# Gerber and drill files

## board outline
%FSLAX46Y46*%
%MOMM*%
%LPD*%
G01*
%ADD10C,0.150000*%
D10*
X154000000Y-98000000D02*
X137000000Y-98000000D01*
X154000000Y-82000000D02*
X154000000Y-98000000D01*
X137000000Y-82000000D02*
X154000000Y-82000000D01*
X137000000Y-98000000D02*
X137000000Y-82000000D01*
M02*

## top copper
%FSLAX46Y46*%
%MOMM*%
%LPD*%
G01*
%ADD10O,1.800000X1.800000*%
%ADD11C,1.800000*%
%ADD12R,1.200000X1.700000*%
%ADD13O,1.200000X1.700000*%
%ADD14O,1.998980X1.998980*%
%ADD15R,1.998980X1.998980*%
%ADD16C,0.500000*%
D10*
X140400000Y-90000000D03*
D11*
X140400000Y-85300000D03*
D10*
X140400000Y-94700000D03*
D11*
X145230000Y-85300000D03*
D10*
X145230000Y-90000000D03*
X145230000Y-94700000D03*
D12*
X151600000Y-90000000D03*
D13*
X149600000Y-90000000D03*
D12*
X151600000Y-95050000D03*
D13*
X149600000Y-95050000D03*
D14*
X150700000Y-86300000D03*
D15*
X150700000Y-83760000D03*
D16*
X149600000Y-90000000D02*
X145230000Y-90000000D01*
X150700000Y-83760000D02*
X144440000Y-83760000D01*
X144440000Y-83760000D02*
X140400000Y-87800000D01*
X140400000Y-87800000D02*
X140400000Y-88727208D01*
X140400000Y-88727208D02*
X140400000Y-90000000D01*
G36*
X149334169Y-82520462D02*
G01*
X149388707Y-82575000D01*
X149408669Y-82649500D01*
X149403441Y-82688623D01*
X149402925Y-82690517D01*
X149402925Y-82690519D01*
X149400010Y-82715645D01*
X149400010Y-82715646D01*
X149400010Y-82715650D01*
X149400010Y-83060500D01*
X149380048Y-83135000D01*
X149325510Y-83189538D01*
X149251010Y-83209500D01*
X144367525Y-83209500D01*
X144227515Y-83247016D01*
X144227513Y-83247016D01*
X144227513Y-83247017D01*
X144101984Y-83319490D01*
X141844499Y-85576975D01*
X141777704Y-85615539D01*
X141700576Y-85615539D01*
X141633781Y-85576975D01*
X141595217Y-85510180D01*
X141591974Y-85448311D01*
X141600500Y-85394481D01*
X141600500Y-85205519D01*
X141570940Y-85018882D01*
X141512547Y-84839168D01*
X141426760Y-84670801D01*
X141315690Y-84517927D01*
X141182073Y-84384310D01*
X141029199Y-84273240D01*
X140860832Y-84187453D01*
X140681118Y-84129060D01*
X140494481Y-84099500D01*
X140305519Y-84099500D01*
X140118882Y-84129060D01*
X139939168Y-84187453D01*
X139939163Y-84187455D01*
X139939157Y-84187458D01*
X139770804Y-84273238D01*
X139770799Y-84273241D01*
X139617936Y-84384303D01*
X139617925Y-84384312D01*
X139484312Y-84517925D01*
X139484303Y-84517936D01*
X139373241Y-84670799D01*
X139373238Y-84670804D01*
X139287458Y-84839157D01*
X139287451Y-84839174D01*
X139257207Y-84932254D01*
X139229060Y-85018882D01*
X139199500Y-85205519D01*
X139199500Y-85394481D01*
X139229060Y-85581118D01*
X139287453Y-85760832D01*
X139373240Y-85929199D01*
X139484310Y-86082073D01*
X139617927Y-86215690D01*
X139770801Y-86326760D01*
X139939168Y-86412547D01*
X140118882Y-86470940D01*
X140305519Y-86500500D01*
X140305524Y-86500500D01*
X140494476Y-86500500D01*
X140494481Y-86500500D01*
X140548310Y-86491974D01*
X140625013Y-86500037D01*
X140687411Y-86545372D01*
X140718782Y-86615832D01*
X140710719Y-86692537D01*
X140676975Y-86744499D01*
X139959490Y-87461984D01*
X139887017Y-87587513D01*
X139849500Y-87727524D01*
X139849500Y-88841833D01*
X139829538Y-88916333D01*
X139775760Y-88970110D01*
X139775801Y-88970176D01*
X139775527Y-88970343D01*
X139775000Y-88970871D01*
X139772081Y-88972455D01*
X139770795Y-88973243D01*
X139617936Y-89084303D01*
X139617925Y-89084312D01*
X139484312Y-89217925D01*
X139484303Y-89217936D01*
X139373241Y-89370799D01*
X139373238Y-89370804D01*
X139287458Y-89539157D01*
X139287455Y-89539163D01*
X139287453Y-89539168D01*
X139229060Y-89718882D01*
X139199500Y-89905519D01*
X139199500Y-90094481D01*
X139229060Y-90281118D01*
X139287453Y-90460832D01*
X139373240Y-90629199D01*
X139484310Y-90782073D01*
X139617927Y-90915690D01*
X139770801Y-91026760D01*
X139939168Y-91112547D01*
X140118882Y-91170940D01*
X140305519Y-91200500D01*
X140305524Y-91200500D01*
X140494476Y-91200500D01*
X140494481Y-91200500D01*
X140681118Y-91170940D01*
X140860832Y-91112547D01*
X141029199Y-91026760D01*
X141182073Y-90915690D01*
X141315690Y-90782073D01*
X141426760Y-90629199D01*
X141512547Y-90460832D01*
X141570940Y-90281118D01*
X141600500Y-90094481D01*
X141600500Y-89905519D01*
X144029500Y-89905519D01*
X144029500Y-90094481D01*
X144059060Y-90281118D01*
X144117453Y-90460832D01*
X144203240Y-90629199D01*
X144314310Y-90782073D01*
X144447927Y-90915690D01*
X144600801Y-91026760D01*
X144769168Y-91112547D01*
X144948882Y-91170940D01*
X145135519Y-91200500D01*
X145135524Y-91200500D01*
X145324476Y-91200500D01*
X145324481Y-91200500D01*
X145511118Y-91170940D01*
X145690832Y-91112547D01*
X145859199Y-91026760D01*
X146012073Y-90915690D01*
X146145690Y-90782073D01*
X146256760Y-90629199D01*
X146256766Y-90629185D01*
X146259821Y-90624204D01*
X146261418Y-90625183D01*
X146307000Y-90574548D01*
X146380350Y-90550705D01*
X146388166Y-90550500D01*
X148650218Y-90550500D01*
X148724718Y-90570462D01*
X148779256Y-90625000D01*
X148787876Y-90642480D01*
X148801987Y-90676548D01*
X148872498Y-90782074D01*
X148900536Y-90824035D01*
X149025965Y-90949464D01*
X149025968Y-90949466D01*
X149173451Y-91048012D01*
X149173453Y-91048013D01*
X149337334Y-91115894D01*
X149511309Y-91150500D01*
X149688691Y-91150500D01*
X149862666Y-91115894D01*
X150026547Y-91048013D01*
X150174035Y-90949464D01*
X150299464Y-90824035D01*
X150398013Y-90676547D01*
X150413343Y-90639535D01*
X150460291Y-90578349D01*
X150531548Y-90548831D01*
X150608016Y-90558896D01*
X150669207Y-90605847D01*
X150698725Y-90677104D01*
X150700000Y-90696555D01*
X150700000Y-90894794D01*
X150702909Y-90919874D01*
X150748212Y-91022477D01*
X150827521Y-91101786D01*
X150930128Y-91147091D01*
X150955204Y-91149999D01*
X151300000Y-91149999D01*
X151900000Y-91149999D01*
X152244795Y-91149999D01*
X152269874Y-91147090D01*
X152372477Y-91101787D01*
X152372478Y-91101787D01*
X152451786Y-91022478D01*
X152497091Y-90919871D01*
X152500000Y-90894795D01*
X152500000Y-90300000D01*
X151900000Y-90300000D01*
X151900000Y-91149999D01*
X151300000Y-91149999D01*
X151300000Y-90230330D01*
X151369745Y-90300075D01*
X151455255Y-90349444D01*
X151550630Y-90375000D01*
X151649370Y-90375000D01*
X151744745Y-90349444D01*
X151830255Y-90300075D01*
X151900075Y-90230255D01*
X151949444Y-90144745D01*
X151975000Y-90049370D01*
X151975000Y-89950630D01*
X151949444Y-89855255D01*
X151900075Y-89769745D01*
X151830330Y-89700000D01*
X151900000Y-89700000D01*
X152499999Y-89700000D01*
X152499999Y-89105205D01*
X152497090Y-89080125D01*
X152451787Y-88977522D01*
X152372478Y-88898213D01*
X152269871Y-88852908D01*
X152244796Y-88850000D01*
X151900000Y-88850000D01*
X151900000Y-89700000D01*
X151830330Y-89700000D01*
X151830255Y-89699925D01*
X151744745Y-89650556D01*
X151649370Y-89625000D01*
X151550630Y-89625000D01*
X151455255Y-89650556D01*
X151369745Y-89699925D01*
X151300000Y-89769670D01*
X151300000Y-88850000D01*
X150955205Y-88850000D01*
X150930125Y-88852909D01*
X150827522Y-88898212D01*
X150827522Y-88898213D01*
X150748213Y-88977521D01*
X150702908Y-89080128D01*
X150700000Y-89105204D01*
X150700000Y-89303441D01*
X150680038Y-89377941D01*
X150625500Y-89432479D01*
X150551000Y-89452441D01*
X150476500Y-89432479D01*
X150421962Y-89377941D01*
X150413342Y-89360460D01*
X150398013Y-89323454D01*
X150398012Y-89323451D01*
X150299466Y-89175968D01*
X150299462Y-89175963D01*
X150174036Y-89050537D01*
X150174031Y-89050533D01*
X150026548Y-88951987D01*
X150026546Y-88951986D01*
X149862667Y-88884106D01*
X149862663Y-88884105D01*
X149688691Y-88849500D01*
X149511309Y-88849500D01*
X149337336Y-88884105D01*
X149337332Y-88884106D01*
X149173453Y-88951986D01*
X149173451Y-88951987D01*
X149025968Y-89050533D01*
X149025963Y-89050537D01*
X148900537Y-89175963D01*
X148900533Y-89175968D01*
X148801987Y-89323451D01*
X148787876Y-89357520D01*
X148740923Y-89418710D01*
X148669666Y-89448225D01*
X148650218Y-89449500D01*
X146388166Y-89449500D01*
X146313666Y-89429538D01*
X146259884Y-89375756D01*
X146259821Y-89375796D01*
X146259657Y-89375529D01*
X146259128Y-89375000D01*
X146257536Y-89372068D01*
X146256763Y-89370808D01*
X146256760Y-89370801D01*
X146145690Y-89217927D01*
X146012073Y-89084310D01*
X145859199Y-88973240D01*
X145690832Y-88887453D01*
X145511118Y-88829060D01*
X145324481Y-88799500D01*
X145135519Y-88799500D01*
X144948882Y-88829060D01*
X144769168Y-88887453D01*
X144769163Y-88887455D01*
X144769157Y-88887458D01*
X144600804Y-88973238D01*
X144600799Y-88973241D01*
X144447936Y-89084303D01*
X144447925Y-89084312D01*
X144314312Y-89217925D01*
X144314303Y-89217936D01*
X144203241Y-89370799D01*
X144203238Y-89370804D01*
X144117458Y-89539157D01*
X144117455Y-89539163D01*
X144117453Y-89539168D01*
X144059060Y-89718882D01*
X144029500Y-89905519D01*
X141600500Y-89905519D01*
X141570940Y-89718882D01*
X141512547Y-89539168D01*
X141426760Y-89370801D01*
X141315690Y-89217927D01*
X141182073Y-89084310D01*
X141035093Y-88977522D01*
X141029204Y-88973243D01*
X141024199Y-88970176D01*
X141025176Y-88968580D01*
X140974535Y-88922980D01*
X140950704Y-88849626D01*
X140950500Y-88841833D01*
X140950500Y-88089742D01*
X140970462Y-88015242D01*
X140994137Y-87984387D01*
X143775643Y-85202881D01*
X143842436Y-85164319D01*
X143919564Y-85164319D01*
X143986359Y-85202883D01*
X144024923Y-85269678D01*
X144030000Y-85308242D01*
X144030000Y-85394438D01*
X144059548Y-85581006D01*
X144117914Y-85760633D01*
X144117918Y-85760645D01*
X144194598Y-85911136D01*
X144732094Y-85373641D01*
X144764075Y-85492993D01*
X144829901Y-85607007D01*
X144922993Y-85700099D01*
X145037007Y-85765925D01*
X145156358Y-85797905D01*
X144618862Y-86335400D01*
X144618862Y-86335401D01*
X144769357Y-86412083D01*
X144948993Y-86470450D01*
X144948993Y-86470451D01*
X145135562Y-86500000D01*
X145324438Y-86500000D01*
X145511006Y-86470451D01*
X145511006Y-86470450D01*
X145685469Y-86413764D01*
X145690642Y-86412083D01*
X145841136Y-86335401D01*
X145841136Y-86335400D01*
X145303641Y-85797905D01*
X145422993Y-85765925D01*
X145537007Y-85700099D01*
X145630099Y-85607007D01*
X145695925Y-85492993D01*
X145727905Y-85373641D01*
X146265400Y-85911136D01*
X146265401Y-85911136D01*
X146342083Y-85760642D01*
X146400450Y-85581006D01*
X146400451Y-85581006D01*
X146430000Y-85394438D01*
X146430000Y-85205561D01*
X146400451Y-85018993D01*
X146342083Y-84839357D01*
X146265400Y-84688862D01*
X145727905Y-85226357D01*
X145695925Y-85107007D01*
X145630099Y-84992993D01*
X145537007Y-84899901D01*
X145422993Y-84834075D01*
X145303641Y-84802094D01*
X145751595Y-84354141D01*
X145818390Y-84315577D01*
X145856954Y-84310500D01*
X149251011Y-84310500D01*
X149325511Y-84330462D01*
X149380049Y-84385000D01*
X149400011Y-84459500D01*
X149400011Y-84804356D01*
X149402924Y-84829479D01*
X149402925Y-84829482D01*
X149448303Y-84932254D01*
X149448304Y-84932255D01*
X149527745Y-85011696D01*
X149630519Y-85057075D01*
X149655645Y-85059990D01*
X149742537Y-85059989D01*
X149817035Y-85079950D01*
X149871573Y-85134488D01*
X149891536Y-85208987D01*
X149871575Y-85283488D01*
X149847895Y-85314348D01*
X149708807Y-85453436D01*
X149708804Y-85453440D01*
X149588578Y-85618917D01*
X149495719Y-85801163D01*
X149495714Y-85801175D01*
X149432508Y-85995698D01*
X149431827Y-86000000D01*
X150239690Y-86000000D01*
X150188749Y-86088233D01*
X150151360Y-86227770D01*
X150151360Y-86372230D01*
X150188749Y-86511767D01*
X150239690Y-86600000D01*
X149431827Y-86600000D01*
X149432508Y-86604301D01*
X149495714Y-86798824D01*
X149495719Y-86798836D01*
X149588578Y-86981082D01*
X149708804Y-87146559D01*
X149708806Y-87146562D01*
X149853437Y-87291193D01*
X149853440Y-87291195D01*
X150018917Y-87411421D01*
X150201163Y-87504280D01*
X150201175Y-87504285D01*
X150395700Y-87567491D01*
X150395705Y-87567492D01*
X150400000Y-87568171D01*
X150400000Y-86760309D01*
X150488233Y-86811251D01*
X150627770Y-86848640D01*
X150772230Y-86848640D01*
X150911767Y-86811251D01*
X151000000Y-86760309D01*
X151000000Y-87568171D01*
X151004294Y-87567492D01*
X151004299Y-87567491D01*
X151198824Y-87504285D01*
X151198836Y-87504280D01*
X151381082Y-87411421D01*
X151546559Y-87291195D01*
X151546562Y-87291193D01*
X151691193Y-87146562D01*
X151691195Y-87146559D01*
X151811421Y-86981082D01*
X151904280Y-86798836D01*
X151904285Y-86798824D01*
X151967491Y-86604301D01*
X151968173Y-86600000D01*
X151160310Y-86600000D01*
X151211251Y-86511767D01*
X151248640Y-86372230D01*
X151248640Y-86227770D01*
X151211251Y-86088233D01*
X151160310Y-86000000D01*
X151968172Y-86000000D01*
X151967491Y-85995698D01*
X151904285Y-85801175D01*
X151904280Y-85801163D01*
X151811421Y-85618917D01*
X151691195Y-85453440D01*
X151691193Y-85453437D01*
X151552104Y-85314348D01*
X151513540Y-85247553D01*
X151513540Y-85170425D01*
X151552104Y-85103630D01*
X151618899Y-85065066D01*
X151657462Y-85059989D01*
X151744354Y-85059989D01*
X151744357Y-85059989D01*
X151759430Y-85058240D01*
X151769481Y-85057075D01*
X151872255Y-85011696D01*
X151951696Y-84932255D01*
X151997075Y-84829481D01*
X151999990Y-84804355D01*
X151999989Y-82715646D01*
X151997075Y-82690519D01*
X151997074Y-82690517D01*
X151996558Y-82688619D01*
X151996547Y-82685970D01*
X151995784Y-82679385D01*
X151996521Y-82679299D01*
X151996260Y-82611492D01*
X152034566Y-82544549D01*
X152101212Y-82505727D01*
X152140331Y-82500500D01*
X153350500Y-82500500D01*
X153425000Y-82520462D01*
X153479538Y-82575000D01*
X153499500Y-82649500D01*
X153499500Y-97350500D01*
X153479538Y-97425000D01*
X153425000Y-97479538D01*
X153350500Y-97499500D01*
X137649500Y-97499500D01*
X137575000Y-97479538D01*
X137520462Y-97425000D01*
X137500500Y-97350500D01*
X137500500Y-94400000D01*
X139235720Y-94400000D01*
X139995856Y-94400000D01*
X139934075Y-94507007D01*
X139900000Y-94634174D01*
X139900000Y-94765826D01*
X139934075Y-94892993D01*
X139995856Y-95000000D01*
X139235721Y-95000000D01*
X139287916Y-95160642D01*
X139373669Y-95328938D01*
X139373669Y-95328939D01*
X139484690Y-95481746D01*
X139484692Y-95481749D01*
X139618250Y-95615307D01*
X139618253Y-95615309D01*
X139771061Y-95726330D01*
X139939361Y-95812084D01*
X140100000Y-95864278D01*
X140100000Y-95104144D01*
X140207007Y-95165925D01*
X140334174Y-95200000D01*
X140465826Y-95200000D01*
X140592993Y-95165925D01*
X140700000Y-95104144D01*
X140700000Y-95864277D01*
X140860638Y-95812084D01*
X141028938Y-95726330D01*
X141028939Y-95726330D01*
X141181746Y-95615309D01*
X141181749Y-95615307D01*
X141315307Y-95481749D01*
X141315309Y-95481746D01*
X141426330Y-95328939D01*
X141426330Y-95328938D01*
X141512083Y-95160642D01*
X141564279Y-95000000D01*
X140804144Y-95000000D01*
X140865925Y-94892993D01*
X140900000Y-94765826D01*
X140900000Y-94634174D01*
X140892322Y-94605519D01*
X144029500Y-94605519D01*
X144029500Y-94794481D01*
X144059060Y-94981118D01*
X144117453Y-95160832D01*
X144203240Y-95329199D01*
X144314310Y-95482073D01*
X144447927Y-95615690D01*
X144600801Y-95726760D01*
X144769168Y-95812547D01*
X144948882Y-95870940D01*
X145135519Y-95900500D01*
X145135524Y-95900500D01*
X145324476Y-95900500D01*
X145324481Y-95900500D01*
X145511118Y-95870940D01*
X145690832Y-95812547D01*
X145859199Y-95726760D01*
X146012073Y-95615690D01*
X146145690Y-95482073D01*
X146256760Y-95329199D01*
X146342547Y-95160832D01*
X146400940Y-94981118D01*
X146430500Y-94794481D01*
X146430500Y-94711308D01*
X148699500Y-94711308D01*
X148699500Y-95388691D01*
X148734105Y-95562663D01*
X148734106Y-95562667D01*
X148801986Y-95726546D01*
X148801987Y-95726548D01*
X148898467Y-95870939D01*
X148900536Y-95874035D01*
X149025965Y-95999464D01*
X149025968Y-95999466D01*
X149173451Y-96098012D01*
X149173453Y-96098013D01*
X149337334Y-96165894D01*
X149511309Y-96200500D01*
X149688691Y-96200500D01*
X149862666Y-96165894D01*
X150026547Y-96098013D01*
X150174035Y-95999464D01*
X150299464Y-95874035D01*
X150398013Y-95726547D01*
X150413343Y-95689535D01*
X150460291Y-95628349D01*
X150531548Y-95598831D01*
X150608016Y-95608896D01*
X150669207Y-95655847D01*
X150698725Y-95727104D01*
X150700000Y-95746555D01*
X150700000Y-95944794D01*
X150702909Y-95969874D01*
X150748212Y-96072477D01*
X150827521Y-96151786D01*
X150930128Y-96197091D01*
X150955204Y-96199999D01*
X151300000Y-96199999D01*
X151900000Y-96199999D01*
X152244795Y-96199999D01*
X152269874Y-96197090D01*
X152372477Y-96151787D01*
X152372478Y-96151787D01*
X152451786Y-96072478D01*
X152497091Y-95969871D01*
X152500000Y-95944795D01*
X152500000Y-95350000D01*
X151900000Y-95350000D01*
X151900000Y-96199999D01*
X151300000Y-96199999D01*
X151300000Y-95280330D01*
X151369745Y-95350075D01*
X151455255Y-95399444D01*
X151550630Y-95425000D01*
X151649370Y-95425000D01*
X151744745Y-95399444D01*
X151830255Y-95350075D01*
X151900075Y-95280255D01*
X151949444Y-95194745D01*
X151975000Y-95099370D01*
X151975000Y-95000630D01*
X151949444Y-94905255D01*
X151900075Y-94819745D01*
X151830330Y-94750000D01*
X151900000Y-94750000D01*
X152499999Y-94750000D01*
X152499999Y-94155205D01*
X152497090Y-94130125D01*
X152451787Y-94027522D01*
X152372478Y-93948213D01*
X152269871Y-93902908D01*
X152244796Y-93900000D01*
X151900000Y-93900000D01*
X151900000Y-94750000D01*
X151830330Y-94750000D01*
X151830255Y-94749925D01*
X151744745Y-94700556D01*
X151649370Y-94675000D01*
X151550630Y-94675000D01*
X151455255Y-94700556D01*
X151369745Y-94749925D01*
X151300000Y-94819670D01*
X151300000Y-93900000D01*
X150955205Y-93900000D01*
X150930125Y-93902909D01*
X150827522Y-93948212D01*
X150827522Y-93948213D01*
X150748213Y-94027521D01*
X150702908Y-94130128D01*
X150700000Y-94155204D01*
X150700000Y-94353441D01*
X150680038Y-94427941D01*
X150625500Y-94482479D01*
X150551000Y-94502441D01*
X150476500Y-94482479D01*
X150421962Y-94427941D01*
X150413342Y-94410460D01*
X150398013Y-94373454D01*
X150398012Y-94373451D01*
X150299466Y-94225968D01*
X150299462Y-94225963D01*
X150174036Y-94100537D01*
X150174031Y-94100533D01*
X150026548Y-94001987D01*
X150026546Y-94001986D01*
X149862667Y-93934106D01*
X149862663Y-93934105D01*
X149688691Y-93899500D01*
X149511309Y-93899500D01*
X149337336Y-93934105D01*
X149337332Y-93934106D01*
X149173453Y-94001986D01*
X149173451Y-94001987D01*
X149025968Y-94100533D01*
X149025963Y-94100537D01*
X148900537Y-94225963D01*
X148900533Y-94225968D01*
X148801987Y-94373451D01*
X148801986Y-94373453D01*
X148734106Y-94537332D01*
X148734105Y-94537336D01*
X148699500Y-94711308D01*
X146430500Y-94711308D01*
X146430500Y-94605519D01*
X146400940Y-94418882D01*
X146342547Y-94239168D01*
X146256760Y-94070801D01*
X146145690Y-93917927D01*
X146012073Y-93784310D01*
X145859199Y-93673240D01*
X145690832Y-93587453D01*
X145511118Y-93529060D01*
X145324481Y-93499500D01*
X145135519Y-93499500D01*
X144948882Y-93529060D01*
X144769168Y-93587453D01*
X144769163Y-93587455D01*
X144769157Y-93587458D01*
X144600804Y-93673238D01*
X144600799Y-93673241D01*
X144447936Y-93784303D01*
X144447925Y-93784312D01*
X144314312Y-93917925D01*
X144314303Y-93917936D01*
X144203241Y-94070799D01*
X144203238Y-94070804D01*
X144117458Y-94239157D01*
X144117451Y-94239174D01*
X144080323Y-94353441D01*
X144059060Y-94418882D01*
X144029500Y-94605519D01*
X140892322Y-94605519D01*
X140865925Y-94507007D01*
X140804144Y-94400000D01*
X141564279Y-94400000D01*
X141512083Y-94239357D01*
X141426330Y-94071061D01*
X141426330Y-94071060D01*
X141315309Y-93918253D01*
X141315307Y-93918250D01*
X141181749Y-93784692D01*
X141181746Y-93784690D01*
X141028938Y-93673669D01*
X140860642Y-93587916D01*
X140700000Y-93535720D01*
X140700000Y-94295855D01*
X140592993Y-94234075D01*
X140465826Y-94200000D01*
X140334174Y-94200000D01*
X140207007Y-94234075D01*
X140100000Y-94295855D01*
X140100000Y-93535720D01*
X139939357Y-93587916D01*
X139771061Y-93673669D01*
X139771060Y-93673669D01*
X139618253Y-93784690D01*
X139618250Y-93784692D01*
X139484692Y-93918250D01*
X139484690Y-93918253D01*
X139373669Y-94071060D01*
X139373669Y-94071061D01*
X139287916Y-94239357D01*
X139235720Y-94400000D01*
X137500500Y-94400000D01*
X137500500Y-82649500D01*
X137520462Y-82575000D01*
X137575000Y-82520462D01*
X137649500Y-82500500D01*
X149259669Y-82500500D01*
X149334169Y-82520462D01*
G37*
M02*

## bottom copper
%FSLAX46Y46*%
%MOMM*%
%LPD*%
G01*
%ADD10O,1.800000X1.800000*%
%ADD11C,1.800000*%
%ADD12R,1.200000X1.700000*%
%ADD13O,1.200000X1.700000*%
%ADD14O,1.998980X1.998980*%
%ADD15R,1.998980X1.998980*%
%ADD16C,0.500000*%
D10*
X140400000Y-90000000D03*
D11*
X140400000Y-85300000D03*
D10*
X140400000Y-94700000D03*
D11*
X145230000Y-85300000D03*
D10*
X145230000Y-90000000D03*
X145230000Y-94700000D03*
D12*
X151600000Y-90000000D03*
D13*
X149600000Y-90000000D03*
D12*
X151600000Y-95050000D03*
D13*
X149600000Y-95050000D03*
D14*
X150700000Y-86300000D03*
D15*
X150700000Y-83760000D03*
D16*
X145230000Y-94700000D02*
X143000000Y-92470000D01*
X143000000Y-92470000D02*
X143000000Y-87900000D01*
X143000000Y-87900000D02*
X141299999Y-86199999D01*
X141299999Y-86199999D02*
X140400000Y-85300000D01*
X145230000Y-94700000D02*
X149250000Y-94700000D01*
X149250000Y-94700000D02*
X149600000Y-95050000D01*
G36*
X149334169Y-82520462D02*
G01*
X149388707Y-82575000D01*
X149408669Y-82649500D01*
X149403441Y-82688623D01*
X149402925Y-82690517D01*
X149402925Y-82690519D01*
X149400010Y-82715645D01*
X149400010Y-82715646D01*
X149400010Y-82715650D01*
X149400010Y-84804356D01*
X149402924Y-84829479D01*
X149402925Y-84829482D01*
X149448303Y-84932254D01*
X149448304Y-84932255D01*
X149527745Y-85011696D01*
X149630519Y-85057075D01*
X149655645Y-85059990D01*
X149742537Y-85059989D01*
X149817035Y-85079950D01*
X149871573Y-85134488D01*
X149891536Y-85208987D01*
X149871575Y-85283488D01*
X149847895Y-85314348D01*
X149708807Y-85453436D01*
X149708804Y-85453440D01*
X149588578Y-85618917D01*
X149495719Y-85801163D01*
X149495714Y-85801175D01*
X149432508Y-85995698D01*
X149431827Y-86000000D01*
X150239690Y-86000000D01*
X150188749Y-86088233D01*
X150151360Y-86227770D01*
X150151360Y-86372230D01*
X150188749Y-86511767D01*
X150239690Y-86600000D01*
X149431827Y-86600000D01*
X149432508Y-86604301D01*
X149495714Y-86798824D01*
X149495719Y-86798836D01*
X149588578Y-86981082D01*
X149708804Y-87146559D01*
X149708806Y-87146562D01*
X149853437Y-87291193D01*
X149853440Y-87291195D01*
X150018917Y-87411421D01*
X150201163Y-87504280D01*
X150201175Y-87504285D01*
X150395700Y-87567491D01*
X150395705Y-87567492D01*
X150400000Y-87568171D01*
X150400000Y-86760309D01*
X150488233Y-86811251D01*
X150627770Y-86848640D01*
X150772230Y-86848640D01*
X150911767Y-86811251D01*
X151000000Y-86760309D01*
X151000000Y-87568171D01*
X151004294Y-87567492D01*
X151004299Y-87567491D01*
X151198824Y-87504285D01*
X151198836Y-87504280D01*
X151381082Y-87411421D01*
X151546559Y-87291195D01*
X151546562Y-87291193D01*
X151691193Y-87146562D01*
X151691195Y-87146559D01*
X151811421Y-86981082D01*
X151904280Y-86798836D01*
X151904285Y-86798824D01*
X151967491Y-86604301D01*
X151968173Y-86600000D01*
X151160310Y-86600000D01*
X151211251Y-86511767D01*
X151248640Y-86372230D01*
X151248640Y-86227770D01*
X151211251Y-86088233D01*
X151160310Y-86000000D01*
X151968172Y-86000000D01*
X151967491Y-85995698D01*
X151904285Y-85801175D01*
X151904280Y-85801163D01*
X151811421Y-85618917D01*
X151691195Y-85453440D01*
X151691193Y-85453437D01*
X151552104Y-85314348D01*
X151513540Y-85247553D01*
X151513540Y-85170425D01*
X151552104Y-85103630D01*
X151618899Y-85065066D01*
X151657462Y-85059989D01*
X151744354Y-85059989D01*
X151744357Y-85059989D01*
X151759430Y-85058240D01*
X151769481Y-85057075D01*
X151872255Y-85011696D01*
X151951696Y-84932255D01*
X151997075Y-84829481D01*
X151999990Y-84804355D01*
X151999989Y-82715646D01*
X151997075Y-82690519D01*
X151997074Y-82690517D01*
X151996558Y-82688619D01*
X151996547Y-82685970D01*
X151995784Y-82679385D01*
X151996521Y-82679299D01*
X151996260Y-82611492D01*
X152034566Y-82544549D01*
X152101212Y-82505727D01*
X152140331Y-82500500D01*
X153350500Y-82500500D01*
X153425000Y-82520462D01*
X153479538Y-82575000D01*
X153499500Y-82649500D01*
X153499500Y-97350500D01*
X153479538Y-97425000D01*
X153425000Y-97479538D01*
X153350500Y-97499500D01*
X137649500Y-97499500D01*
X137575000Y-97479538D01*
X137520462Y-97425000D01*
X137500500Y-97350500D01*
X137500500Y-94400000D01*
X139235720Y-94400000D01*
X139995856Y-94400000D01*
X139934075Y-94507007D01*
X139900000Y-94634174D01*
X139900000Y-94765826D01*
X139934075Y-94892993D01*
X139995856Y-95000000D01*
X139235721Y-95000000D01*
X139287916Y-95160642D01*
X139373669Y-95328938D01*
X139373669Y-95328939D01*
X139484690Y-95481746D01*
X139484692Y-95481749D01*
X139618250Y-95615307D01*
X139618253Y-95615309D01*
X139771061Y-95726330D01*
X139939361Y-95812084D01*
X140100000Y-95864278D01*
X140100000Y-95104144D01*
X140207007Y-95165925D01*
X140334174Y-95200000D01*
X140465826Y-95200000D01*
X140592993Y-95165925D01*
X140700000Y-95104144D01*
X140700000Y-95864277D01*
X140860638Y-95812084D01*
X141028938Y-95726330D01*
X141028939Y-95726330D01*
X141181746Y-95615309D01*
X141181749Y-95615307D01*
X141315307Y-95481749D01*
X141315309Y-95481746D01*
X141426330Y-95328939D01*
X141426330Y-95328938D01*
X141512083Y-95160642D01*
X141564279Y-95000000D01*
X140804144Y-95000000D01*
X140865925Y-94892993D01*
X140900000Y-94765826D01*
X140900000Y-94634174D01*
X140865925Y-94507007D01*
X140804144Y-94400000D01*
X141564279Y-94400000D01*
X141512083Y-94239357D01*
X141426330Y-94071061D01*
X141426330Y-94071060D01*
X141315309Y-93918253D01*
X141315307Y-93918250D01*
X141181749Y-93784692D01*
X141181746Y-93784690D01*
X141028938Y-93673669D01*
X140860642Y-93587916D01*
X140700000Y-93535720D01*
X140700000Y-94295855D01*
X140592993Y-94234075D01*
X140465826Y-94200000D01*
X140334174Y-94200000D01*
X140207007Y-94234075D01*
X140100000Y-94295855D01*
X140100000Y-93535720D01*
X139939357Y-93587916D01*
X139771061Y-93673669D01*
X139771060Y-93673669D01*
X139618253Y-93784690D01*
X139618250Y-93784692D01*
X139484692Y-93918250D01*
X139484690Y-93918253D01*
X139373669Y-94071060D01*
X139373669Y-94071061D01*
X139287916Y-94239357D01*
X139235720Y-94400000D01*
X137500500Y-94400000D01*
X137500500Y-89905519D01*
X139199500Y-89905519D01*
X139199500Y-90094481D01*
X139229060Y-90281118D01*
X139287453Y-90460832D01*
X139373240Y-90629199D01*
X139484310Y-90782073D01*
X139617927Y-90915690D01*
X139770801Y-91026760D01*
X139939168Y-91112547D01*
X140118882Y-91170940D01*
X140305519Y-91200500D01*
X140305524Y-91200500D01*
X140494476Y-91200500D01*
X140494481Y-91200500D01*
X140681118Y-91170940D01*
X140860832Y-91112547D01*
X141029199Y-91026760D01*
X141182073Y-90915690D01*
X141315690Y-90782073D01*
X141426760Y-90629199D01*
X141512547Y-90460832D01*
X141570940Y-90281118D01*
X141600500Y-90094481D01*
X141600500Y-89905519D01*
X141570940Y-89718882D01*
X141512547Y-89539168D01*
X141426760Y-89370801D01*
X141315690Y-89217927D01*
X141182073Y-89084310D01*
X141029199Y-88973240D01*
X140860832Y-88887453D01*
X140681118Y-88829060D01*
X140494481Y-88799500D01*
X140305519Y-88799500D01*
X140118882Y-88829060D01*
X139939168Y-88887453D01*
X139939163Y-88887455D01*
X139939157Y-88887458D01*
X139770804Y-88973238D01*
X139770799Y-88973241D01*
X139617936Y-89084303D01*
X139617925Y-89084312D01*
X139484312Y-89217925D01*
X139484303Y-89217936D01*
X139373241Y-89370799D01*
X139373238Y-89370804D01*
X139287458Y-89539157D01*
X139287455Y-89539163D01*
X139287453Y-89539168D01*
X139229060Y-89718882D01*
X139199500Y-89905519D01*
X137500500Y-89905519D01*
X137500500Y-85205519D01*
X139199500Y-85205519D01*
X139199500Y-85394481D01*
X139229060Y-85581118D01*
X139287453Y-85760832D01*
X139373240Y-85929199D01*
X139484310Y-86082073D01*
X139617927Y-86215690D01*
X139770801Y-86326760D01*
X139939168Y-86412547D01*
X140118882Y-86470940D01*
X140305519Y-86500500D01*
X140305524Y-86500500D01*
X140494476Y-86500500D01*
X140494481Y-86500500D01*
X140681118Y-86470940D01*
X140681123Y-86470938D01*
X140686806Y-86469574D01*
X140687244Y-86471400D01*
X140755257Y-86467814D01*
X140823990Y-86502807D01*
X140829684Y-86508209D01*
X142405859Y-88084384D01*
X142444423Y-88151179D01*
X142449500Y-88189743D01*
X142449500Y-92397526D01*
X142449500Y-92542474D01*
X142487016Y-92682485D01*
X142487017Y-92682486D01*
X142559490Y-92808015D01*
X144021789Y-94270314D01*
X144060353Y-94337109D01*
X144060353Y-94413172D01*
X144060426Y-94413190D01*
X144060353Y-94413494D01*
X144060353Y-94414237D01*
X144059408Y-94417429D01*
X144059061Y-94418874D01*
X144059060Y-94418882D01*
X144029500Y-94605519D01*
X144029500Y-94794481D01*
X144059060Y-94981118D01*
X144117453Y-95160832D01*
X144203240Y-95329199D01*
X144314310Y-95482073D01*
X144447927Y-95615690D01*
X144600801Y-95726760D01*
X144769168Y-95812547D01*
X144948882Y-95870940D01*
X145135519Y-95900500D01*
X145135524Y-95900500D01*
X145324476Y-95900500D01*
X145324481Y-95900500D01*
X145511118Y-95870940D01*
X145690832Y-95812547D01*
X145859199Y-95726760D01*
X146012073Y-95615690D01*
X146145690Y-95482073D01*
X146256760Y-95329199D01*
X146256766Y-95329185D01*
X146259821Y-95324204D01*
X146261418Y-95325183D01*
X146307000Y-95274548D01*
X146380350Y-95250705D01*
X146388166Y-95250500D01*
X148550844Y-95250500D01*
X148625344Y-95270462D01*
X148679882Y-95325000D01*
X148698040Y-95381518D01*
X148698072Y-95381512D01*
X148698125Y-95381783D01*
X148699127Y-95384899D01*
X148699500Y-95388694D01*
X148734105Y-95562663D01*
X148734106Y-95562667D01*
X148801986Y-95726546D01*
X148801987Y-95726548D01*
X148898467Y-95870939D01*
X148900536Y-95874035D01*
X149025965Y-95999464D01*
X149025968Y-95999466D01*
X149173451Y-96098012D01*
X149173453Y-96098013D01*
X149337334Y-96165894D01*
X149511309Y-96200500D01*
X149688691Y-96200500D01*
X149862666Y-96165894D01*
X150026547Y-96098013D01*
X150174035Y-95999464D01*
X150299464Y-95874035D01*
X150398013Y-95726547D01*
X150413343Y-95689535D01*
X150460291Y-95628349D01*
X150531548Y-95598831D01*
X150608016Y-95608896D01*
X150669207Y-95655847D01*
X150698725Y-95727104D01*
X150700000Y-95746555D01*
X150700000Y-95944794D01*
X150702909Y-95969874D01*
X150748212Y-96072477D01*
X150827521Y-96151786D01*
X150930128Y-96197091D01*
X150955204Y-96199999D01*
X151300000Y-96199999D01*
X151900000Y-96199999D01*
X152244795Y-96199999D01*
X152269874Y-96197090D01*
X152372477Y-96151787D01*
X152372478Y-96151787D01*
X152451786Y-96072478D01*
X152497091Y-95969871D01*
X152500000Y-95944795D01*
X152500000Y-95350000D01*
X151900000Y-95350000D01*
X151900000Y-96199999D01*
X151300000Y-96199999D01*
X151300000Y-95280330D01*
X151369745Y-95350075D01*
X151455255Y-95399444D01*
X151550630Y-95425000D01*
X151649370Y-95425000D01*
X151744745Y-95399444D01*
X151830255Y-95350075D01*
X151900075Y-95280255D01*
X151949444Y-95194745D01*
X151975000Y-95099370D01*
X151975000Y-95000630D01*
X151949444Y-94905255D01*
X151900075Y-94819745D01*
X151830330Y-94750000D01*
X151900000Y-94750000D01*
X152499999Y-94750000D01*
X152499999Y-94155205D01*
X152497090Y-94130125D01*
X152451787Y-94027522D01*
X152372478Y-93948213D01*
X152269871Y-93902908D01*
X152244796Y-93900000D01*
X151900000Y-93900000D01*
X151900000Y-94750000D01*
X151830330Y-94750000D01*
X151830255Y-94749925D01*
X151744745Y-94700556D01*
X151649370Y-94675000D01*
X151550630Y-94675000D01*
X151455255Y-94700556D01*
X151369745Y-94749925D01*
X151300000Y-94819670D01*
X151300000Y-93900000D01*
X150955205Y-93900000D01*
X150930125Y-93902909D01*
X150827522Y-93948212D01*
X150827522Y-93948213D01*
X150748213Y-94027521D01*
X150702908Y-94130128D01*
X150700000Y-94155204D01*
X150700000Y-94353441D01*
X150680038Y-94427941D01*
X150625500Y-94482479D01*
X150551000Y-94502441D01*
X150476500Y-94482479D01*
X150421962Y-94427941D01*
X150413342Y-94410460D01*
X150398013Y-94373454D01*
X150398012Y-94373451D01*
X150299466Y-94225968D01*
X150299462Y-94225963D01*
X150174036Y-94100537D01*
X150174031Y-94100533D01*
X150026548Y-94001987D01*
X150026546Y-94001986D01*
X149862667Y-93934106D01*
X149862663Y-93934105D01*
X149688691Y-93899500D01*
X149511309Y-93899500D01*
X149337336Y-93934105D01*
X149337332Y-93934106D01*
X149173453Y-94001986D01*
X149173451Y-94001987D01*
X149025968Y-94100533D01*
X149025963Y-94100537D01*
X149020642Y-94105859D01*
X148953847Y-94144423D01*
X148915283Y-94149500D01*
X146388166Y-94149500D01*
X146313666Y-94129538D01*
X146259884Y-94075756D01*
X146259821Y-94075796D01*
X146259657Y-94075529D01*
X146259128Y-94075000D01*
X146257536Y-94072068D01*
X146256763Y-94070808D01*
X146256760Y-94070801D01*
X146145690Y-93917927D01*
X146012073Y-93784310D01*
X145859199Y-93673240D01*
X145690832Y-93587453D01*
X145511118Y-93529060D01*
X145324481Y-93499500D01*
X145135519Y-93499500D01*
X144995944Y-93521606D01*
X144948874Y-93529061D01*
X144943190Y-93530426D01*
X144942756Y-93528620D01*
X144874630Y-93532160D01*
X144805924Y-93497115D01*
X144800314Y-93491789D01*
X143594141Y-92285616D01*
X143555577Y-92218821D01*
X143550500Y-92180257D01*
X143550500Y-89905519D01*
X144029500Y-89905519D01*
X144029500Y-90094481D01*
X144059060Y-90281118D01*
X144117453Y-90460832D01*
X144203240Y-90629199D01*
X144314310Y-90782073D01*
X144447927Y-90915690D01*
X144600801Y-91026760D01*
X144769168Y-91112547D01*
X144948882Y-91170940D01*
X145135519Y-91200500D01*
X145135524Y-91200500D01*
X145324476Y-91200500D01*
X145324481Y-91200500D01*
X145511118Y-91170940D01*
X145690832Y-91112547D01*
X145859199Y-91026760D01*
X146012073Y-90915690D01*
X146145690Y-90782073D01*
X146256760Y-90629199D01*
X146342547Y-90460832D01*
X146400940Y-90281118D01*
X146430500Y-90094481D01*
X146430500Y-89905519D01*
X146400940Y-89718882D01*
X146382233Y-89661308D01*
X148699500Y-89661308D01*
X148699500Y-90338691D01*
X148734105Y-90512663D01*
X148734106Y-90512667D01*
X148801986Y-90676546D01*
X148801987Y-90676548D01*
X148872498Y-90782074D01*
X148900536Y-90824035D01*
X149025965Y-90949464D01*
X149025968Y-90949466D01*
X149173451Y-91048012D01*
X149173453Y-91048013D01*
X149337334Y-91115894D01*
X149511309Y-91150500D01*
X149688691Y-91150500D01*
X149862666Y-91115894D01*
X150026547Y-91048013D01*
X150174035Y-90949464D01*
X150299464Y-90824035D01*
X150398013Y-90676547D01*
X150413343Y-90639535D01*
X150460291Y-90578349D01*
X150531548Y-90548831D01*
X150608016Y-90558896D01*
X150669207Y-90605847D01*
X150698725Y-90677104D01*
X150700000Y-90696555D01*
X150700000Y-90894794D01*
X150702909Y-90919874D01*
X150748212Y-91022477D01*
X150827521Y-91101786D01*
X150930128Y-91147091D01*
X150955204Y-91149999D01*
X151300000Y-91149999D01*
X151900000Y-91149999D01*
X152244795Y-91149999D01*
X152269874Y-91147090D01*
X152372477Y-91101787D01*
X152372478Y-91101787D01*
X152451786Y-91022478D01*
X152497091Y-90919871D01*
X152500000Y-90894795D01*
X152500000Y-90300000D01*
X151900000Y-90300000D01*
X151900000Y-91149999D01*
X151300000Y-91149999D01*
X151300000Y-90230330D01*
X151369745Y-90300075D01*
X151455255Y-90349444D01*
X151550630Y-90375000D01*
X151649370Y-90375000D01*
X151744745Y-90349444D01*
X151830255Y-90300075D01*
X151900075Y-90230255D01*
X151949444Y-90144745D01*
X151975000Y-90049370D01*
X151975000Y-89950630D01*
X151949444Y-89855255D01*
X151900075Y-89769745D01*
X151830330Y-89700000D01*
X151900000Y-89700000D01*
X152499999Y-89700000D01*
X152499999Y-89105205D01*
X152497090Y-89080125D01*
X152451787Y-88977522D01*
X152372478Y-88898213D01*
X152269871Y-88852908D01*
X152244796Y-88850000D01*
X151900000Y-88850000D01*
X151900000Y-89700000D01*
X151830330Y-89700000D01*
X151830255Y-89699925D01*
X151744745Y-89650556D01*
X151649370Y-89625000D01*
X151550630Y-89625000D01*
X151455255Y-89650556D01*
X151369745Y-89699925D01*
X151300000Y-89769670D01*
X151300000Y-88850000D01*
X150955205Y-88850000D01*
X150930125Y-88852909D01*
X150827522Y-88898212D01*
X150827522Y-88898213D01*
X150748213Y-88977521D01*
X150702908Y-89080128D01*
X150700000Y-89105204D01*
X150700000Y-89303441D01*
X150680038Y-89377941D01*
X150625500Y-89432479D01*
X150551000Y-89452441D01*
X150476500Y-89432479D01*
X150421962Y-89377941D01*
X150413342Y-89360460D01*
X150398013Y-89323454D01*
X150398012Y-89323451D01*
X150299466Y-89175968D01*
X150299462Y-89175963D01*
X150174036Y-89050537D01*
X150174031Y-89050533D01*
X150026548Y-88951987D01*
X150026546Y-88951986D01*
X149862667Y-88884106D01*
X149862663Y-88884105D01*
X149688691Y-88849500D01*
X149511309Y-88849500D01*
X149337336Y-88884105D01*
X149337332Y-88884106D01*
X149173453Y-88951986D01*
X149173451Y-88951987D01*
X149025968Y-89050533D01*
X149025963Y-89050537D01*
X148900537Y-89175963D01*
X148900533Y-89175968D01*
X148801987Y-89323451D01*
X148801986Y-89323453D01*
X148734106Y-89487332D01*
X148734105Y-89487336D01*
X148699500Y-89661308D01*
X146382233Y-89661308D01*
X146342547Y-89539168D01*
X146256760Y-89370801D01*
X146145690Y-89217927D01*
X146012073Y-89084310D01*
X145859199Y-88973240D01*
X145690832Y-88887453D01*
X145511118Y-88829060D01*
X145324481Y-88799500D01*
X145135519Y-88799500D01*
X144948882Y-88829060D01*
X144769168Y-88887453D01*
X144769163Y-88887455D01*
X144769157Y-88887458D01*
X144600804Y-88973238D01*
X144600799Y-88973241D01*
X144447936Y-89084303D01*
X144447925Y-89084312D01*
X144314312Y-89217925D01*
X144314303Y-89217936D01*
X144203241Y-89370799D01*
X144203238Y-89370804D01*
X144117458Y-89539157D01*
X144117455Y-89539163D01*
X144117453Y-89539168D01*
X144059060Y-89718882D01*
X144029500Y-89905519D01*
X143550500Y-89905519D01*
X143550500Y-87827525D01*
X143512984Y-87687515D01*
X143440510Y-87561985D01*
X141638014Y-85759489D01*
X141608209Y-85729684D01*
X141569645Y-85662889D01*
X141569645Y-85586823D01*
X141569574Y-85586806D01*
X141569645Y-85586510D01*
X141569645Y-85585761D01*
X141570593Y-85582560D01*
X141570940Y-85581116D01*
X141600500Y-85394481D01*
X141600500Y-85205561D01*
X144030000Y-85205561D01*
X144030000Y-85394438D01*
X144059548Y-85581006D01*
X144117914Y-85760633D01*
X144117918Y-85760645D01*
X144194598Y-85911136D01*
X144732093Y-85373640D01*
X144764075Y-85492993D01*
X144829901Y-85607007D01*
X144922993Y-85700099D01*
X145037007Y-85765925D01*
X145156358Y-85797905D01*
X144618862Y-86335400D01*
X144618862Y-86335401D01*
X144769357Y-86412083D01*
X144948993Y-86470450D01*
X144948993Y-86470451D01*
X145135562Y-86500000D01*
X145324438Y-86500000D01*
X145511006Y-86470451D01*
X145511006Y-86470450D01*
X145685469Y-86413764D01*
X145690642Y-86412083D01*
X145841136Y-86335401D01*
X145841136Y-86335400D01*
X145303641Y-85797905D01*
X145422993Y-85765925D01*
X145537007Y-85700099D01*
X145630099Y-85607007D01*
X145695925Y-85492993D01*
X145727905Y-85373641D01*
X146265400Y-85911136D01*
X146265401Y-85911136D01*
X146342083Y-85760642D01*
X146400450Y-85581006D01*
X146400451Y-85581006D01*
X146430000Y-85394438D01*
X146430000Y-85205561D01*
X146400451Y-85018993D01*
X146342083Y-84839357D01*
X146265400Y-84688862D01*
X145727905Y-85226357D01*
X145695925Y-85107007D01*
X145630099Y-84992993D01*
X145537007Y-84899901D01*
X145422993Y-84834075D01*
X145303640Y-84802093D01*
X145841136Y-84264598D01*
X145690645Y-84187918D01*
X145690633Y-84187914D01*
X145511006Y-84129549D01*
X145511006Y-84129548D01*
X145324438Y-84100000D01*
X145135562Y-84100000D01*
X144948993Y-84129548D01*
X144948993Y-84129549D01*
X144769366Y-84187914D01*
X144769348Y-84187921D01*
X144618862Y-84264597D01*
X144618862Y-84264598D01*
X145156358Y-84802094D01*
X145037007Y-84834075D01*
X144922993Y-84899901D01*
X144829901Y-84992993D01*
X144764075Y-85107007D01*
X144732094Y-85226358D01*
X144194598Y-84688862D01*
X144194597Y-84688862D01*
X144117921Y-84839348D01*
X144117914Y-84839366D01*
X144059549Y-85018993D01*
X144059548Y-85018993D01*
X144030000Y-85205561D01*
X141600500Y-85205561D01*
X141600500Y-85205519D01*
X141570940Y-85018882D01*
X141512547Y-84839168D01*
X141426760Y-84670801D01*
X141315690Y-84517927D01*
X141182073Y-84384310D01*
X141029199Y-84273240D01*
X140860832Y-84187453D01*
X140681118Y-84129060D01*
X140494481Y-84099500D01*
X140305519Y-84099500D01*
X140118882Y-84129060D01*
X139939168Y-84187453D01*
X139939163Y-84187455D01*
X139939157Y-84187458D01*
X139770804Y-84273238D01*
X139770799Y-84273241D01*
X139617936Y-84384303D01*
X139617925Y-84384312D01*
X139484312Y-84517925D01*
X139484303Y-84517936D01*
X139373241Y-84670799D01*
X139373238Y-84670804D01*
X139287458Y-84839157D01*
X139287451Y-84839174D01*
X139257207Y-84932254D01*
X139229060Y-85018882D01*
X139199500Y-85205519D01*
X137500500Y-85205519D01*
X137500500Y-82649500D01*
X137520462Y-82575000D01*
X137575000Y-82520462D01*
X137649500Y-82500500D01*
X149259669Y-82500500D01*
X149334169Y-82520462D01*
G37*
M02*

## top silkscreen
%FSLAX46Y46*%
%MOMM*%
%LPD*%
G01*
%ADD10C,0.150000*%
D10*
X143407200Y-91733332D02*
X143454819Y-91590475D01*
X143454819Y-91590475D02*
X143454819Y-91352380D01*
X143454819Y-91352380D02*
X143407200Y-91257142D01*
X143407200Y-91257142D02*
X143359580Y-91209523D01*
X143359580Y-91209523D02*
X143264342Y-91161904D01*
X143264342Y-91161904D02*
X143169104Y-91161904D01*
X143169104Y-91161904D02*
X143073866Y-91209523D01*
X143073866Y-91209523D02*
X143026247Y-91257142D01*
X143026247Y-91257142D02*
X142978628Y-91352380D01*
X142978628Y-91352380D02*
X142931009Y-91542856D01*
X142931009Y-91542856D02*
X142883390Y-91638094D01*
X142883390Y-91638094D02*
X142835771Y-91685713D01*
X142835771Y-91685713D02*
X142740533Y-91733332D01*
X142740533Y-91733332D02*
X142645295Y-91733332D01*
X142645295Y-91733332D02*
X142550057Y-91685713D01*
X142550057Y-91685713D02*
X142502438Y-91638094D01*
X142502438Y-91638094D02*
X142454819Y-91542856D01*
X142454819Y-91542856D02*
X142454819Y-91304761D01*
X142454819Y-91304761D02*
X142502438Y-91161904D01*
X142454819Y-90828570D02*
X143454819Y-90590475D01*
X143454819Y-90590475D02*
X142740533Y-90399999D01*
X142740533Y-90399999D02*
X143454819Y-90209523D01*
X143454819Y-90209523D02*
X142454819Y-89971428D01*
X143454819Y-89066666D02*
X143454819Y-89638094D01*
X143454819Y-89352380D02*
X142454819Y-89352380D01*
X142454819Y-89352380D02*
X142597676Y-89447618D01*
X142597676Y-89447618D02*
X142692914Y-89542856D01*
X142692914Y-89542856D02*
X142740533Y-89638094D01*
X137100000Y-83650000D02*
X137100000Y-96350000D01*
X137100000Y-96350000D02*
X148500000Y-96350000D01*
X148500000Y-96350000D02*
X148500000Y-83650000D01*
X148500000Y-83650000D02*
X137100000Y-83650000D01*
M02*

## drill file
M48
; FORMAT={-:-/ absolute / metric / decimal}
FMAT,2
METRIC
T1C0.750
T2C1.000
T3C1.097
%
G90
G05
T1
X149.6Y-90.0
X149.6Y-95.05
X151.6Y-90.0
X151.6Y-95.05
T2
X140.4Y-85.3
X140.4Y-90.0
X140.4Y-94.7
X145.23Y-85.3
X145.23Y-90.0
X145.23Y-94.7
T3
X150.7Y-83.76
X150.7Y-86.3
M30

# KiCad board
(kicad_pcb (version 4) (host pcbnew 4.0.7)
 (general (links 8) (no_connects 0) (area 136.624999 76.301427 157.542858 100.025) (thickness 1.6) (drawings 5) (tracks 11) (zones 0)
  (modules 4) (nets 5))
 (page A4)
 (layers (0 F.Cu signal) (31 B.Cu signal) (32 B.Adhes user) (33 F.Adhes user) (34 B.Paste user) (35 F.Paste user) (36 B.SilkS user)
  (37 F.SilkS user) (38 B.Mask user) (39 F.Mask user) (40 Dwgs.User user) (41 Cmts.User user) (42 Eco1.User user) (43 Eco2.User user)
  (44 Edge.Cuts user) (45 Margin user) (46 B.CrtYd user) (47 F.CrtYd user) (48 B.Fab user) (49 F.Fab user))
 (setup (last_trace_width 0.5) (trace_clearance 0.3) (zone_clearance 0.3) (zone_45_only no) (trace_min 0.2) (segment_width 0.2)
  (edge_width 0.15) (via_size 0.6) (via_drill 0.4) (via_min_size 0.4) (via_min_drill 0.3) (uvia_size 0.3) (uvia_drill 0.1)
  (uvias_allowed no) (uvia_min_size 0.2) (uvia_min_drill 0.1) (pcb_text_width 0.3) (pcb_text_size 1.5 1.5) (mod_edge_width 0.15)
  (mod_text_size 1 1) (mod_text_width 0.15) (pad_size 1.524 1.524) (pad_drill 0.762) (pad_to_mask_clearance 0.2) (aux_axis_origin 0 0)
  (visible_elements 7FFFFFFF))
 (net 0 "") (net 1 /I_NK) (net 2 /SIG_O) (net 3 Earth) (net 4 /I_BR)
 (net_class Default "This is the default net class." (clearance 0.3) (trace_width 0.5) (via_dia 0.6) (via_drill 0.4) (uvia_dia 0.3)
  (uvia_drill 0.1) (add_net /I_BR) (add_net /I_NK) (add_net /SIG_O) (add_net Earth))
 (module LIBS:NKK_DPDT (layer F.Cu) (at 145.2 85.3 90)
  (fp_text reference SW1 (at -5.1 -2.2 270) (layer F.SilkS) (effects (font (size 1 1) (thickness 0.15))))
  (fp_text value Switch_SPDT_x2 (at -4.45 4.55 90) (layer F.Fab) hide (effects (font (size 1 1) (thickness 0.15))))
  (fp_line (start 1.65 -8.1) (end -11.05 -8.1) (layer F.SilkS) (width 0.15))
  (fp_line (start -11.05 -8.1) (end -11.05 3.3) (layer F.SilkS) (width 0.15))
  (fp_line (start -11.05 3.3) (end 1.65 3.3) (layer F.SilkS) (width 0.15))
  (fp_line (start 1.65 3.3) (end 1.65 -8.1) (layer F.SilkS) (width 0.15))
  (pad 5 thru_hole oval (at -4.7 -4.8 270) (size 1.8 1.8) (drill 1) (layers *.Cu *.Mask) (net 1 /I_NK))
  (pad 4 thru_hole circle (at 0 -4.8 270) (size 1.8 1.8) (drill 1) (layers *.Cu *.Mask) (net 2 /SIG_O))
  (pad 6 thru_hole oval (at -9.4 -4.8 270) (size 1.8 1.8) (drill 1) (layers *.Cu *.Mask) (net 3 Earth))
  (pad 1 thru_hole circle (at 0 0.03 270) (size 1.8 1.8) (drill 1) (layers *.Cu *.Mask) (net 3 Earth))
  (pad 2 thru_hole oval (at -4.7 0.03 270) (size 1.8 1.8) (drill 1) (layers *.Cu *.Mask) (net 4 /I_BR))
  (pad 3 thru_hole oval (at -9.4 0.03 270) (size 1.8 1.8) (drill 1) (layers *.Cu *.Mask) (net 2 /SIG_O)))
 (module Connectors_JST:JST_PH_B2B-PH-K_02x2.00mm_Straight (layer B.Cu) (at 151.6 90 180)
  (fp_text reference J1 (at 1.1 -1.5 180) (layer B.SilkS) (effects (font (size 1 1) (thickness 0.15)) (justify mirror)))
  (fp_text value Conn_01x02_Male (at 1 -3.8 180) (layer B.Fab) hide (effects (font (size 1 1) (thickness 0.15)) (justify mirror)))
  (pad 1 thru_hole rect (at 0 0 180) (size 1.2 1.7) (drill 0.75) (layers *.Cu *.Mask) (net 3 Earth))
  (pad 2 thru_hole oval (at 2 0 180) (size 1.2 1.7) (drill 0.75) (layers *.Cu *.Mask) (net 4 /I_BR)))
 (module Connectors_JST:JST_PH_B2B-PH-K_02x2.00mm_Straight (layer B.Cu) (at 151.6 95.05 180)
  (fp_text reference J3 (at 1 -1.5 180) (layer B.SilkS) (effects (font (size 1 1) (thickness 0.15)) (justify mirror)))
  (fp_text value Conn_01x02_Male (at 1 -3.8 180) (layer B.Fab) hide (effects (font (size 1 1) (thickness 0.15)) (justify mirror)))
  (pad 1 thru_hole rect (at 0 0 180) (size 1.2 1.7) (drill 0.75) (layers *.Cu *.Mask) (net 3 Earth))
  (pad 2 thru_hole oval (at 2 0 180) (size 1.2 1.7) (drill 0.75) (layers *.Cu *.Mask) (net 2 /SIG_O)))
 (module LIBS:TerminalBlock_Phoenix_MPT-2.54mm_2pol (layer B.Cu) (at 150.7 83.76 270)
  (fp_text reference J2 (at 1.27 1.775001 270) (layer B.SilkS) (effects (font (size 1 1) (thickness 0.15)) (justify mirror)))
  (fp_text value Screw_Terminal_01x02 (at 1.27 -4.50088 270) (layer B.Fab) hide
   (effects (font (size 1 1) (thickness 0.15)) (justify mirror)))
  (pad 2 thru_hole oval (at 2.54 0 270) (size 1.99898 1.99898) (drill 1.09728) (layers *.Cu *.Mask) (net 3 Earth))
  (pad 1 thru_hole rect (at 0 0 270) (size 1.99898 1.99898) (drill 1.09728) (layers *.Cu *.Mask) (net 1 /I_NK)))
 (gr_line (start 154 98) (end 137 98) (layer Edge.Cuts) (width 0.15))
 (gr_line (start 154 82) (end 154 98) (layer Edge.Cuts) (width 0.15))
 (gr_line (start 137 82) (end 154 82) (layer Edge.Cuts) (width 0.15))
 (gr_line (start 137 98) (end 137 82) (layer Edge.Cuts) (width 0.15))
 (segment (start 145.23 94.7) (end 143 92.47) (width 0.5) (layer B.Cu) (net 2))
 (segment (start 143 92.47) (end 143 87.9) (width 0.5) (layer B.Cu) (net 2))
 (segment (start 143 87.9) (end 141.299999 86.199999) (width 0.5) (layer B.Cu) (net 2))
 (segment (start 141.299999 86.199999) (end 140.4 85.3) (width 0.5) (layer B.Cu) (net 2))
 (segment (start 145.23 94.7) (end 149.25 94.7) (width 0.5) (layer B.Cu) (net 2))
 (segment (start 149.25 94.7) (end 149.6 95.05) (width 0.5) (layer B.Cu) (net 2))
 (segment (start 149.6 90) (end 145.23 90) (width 0.5) (layer F.Cu) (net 4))
 (segment (start 150.7 83.76) (end 144.44 83.76) (width 0.5) (layer F.Cu) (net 1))
 (segment (start 144.44 83.76) (end 140.4 87.8) (width 0.5) (layer F.Cu) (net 1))
 (segment (start 140.4 87.8) (end 140.4 88.727208) (width 0.5) (layer F.Cu) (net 1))
 (segment (start 140.4 88.727208) (end 140.4 90) (width 0.5) (layer F.Cu) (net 1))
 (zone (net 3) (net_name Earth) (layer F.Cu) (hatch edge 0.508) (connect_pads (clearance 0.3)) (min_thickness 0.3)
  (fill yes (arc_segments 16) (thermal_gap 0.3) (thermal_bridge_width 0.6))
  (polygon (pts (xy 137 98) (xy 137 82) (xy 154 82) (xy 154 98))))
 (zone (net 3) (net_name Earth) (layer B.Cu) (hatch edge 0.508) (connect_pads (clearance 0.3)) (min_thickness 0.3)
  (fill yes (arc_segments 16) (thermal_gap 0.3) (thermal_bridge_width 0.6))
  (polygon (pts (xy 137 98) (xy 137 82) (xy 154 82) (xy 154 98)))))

